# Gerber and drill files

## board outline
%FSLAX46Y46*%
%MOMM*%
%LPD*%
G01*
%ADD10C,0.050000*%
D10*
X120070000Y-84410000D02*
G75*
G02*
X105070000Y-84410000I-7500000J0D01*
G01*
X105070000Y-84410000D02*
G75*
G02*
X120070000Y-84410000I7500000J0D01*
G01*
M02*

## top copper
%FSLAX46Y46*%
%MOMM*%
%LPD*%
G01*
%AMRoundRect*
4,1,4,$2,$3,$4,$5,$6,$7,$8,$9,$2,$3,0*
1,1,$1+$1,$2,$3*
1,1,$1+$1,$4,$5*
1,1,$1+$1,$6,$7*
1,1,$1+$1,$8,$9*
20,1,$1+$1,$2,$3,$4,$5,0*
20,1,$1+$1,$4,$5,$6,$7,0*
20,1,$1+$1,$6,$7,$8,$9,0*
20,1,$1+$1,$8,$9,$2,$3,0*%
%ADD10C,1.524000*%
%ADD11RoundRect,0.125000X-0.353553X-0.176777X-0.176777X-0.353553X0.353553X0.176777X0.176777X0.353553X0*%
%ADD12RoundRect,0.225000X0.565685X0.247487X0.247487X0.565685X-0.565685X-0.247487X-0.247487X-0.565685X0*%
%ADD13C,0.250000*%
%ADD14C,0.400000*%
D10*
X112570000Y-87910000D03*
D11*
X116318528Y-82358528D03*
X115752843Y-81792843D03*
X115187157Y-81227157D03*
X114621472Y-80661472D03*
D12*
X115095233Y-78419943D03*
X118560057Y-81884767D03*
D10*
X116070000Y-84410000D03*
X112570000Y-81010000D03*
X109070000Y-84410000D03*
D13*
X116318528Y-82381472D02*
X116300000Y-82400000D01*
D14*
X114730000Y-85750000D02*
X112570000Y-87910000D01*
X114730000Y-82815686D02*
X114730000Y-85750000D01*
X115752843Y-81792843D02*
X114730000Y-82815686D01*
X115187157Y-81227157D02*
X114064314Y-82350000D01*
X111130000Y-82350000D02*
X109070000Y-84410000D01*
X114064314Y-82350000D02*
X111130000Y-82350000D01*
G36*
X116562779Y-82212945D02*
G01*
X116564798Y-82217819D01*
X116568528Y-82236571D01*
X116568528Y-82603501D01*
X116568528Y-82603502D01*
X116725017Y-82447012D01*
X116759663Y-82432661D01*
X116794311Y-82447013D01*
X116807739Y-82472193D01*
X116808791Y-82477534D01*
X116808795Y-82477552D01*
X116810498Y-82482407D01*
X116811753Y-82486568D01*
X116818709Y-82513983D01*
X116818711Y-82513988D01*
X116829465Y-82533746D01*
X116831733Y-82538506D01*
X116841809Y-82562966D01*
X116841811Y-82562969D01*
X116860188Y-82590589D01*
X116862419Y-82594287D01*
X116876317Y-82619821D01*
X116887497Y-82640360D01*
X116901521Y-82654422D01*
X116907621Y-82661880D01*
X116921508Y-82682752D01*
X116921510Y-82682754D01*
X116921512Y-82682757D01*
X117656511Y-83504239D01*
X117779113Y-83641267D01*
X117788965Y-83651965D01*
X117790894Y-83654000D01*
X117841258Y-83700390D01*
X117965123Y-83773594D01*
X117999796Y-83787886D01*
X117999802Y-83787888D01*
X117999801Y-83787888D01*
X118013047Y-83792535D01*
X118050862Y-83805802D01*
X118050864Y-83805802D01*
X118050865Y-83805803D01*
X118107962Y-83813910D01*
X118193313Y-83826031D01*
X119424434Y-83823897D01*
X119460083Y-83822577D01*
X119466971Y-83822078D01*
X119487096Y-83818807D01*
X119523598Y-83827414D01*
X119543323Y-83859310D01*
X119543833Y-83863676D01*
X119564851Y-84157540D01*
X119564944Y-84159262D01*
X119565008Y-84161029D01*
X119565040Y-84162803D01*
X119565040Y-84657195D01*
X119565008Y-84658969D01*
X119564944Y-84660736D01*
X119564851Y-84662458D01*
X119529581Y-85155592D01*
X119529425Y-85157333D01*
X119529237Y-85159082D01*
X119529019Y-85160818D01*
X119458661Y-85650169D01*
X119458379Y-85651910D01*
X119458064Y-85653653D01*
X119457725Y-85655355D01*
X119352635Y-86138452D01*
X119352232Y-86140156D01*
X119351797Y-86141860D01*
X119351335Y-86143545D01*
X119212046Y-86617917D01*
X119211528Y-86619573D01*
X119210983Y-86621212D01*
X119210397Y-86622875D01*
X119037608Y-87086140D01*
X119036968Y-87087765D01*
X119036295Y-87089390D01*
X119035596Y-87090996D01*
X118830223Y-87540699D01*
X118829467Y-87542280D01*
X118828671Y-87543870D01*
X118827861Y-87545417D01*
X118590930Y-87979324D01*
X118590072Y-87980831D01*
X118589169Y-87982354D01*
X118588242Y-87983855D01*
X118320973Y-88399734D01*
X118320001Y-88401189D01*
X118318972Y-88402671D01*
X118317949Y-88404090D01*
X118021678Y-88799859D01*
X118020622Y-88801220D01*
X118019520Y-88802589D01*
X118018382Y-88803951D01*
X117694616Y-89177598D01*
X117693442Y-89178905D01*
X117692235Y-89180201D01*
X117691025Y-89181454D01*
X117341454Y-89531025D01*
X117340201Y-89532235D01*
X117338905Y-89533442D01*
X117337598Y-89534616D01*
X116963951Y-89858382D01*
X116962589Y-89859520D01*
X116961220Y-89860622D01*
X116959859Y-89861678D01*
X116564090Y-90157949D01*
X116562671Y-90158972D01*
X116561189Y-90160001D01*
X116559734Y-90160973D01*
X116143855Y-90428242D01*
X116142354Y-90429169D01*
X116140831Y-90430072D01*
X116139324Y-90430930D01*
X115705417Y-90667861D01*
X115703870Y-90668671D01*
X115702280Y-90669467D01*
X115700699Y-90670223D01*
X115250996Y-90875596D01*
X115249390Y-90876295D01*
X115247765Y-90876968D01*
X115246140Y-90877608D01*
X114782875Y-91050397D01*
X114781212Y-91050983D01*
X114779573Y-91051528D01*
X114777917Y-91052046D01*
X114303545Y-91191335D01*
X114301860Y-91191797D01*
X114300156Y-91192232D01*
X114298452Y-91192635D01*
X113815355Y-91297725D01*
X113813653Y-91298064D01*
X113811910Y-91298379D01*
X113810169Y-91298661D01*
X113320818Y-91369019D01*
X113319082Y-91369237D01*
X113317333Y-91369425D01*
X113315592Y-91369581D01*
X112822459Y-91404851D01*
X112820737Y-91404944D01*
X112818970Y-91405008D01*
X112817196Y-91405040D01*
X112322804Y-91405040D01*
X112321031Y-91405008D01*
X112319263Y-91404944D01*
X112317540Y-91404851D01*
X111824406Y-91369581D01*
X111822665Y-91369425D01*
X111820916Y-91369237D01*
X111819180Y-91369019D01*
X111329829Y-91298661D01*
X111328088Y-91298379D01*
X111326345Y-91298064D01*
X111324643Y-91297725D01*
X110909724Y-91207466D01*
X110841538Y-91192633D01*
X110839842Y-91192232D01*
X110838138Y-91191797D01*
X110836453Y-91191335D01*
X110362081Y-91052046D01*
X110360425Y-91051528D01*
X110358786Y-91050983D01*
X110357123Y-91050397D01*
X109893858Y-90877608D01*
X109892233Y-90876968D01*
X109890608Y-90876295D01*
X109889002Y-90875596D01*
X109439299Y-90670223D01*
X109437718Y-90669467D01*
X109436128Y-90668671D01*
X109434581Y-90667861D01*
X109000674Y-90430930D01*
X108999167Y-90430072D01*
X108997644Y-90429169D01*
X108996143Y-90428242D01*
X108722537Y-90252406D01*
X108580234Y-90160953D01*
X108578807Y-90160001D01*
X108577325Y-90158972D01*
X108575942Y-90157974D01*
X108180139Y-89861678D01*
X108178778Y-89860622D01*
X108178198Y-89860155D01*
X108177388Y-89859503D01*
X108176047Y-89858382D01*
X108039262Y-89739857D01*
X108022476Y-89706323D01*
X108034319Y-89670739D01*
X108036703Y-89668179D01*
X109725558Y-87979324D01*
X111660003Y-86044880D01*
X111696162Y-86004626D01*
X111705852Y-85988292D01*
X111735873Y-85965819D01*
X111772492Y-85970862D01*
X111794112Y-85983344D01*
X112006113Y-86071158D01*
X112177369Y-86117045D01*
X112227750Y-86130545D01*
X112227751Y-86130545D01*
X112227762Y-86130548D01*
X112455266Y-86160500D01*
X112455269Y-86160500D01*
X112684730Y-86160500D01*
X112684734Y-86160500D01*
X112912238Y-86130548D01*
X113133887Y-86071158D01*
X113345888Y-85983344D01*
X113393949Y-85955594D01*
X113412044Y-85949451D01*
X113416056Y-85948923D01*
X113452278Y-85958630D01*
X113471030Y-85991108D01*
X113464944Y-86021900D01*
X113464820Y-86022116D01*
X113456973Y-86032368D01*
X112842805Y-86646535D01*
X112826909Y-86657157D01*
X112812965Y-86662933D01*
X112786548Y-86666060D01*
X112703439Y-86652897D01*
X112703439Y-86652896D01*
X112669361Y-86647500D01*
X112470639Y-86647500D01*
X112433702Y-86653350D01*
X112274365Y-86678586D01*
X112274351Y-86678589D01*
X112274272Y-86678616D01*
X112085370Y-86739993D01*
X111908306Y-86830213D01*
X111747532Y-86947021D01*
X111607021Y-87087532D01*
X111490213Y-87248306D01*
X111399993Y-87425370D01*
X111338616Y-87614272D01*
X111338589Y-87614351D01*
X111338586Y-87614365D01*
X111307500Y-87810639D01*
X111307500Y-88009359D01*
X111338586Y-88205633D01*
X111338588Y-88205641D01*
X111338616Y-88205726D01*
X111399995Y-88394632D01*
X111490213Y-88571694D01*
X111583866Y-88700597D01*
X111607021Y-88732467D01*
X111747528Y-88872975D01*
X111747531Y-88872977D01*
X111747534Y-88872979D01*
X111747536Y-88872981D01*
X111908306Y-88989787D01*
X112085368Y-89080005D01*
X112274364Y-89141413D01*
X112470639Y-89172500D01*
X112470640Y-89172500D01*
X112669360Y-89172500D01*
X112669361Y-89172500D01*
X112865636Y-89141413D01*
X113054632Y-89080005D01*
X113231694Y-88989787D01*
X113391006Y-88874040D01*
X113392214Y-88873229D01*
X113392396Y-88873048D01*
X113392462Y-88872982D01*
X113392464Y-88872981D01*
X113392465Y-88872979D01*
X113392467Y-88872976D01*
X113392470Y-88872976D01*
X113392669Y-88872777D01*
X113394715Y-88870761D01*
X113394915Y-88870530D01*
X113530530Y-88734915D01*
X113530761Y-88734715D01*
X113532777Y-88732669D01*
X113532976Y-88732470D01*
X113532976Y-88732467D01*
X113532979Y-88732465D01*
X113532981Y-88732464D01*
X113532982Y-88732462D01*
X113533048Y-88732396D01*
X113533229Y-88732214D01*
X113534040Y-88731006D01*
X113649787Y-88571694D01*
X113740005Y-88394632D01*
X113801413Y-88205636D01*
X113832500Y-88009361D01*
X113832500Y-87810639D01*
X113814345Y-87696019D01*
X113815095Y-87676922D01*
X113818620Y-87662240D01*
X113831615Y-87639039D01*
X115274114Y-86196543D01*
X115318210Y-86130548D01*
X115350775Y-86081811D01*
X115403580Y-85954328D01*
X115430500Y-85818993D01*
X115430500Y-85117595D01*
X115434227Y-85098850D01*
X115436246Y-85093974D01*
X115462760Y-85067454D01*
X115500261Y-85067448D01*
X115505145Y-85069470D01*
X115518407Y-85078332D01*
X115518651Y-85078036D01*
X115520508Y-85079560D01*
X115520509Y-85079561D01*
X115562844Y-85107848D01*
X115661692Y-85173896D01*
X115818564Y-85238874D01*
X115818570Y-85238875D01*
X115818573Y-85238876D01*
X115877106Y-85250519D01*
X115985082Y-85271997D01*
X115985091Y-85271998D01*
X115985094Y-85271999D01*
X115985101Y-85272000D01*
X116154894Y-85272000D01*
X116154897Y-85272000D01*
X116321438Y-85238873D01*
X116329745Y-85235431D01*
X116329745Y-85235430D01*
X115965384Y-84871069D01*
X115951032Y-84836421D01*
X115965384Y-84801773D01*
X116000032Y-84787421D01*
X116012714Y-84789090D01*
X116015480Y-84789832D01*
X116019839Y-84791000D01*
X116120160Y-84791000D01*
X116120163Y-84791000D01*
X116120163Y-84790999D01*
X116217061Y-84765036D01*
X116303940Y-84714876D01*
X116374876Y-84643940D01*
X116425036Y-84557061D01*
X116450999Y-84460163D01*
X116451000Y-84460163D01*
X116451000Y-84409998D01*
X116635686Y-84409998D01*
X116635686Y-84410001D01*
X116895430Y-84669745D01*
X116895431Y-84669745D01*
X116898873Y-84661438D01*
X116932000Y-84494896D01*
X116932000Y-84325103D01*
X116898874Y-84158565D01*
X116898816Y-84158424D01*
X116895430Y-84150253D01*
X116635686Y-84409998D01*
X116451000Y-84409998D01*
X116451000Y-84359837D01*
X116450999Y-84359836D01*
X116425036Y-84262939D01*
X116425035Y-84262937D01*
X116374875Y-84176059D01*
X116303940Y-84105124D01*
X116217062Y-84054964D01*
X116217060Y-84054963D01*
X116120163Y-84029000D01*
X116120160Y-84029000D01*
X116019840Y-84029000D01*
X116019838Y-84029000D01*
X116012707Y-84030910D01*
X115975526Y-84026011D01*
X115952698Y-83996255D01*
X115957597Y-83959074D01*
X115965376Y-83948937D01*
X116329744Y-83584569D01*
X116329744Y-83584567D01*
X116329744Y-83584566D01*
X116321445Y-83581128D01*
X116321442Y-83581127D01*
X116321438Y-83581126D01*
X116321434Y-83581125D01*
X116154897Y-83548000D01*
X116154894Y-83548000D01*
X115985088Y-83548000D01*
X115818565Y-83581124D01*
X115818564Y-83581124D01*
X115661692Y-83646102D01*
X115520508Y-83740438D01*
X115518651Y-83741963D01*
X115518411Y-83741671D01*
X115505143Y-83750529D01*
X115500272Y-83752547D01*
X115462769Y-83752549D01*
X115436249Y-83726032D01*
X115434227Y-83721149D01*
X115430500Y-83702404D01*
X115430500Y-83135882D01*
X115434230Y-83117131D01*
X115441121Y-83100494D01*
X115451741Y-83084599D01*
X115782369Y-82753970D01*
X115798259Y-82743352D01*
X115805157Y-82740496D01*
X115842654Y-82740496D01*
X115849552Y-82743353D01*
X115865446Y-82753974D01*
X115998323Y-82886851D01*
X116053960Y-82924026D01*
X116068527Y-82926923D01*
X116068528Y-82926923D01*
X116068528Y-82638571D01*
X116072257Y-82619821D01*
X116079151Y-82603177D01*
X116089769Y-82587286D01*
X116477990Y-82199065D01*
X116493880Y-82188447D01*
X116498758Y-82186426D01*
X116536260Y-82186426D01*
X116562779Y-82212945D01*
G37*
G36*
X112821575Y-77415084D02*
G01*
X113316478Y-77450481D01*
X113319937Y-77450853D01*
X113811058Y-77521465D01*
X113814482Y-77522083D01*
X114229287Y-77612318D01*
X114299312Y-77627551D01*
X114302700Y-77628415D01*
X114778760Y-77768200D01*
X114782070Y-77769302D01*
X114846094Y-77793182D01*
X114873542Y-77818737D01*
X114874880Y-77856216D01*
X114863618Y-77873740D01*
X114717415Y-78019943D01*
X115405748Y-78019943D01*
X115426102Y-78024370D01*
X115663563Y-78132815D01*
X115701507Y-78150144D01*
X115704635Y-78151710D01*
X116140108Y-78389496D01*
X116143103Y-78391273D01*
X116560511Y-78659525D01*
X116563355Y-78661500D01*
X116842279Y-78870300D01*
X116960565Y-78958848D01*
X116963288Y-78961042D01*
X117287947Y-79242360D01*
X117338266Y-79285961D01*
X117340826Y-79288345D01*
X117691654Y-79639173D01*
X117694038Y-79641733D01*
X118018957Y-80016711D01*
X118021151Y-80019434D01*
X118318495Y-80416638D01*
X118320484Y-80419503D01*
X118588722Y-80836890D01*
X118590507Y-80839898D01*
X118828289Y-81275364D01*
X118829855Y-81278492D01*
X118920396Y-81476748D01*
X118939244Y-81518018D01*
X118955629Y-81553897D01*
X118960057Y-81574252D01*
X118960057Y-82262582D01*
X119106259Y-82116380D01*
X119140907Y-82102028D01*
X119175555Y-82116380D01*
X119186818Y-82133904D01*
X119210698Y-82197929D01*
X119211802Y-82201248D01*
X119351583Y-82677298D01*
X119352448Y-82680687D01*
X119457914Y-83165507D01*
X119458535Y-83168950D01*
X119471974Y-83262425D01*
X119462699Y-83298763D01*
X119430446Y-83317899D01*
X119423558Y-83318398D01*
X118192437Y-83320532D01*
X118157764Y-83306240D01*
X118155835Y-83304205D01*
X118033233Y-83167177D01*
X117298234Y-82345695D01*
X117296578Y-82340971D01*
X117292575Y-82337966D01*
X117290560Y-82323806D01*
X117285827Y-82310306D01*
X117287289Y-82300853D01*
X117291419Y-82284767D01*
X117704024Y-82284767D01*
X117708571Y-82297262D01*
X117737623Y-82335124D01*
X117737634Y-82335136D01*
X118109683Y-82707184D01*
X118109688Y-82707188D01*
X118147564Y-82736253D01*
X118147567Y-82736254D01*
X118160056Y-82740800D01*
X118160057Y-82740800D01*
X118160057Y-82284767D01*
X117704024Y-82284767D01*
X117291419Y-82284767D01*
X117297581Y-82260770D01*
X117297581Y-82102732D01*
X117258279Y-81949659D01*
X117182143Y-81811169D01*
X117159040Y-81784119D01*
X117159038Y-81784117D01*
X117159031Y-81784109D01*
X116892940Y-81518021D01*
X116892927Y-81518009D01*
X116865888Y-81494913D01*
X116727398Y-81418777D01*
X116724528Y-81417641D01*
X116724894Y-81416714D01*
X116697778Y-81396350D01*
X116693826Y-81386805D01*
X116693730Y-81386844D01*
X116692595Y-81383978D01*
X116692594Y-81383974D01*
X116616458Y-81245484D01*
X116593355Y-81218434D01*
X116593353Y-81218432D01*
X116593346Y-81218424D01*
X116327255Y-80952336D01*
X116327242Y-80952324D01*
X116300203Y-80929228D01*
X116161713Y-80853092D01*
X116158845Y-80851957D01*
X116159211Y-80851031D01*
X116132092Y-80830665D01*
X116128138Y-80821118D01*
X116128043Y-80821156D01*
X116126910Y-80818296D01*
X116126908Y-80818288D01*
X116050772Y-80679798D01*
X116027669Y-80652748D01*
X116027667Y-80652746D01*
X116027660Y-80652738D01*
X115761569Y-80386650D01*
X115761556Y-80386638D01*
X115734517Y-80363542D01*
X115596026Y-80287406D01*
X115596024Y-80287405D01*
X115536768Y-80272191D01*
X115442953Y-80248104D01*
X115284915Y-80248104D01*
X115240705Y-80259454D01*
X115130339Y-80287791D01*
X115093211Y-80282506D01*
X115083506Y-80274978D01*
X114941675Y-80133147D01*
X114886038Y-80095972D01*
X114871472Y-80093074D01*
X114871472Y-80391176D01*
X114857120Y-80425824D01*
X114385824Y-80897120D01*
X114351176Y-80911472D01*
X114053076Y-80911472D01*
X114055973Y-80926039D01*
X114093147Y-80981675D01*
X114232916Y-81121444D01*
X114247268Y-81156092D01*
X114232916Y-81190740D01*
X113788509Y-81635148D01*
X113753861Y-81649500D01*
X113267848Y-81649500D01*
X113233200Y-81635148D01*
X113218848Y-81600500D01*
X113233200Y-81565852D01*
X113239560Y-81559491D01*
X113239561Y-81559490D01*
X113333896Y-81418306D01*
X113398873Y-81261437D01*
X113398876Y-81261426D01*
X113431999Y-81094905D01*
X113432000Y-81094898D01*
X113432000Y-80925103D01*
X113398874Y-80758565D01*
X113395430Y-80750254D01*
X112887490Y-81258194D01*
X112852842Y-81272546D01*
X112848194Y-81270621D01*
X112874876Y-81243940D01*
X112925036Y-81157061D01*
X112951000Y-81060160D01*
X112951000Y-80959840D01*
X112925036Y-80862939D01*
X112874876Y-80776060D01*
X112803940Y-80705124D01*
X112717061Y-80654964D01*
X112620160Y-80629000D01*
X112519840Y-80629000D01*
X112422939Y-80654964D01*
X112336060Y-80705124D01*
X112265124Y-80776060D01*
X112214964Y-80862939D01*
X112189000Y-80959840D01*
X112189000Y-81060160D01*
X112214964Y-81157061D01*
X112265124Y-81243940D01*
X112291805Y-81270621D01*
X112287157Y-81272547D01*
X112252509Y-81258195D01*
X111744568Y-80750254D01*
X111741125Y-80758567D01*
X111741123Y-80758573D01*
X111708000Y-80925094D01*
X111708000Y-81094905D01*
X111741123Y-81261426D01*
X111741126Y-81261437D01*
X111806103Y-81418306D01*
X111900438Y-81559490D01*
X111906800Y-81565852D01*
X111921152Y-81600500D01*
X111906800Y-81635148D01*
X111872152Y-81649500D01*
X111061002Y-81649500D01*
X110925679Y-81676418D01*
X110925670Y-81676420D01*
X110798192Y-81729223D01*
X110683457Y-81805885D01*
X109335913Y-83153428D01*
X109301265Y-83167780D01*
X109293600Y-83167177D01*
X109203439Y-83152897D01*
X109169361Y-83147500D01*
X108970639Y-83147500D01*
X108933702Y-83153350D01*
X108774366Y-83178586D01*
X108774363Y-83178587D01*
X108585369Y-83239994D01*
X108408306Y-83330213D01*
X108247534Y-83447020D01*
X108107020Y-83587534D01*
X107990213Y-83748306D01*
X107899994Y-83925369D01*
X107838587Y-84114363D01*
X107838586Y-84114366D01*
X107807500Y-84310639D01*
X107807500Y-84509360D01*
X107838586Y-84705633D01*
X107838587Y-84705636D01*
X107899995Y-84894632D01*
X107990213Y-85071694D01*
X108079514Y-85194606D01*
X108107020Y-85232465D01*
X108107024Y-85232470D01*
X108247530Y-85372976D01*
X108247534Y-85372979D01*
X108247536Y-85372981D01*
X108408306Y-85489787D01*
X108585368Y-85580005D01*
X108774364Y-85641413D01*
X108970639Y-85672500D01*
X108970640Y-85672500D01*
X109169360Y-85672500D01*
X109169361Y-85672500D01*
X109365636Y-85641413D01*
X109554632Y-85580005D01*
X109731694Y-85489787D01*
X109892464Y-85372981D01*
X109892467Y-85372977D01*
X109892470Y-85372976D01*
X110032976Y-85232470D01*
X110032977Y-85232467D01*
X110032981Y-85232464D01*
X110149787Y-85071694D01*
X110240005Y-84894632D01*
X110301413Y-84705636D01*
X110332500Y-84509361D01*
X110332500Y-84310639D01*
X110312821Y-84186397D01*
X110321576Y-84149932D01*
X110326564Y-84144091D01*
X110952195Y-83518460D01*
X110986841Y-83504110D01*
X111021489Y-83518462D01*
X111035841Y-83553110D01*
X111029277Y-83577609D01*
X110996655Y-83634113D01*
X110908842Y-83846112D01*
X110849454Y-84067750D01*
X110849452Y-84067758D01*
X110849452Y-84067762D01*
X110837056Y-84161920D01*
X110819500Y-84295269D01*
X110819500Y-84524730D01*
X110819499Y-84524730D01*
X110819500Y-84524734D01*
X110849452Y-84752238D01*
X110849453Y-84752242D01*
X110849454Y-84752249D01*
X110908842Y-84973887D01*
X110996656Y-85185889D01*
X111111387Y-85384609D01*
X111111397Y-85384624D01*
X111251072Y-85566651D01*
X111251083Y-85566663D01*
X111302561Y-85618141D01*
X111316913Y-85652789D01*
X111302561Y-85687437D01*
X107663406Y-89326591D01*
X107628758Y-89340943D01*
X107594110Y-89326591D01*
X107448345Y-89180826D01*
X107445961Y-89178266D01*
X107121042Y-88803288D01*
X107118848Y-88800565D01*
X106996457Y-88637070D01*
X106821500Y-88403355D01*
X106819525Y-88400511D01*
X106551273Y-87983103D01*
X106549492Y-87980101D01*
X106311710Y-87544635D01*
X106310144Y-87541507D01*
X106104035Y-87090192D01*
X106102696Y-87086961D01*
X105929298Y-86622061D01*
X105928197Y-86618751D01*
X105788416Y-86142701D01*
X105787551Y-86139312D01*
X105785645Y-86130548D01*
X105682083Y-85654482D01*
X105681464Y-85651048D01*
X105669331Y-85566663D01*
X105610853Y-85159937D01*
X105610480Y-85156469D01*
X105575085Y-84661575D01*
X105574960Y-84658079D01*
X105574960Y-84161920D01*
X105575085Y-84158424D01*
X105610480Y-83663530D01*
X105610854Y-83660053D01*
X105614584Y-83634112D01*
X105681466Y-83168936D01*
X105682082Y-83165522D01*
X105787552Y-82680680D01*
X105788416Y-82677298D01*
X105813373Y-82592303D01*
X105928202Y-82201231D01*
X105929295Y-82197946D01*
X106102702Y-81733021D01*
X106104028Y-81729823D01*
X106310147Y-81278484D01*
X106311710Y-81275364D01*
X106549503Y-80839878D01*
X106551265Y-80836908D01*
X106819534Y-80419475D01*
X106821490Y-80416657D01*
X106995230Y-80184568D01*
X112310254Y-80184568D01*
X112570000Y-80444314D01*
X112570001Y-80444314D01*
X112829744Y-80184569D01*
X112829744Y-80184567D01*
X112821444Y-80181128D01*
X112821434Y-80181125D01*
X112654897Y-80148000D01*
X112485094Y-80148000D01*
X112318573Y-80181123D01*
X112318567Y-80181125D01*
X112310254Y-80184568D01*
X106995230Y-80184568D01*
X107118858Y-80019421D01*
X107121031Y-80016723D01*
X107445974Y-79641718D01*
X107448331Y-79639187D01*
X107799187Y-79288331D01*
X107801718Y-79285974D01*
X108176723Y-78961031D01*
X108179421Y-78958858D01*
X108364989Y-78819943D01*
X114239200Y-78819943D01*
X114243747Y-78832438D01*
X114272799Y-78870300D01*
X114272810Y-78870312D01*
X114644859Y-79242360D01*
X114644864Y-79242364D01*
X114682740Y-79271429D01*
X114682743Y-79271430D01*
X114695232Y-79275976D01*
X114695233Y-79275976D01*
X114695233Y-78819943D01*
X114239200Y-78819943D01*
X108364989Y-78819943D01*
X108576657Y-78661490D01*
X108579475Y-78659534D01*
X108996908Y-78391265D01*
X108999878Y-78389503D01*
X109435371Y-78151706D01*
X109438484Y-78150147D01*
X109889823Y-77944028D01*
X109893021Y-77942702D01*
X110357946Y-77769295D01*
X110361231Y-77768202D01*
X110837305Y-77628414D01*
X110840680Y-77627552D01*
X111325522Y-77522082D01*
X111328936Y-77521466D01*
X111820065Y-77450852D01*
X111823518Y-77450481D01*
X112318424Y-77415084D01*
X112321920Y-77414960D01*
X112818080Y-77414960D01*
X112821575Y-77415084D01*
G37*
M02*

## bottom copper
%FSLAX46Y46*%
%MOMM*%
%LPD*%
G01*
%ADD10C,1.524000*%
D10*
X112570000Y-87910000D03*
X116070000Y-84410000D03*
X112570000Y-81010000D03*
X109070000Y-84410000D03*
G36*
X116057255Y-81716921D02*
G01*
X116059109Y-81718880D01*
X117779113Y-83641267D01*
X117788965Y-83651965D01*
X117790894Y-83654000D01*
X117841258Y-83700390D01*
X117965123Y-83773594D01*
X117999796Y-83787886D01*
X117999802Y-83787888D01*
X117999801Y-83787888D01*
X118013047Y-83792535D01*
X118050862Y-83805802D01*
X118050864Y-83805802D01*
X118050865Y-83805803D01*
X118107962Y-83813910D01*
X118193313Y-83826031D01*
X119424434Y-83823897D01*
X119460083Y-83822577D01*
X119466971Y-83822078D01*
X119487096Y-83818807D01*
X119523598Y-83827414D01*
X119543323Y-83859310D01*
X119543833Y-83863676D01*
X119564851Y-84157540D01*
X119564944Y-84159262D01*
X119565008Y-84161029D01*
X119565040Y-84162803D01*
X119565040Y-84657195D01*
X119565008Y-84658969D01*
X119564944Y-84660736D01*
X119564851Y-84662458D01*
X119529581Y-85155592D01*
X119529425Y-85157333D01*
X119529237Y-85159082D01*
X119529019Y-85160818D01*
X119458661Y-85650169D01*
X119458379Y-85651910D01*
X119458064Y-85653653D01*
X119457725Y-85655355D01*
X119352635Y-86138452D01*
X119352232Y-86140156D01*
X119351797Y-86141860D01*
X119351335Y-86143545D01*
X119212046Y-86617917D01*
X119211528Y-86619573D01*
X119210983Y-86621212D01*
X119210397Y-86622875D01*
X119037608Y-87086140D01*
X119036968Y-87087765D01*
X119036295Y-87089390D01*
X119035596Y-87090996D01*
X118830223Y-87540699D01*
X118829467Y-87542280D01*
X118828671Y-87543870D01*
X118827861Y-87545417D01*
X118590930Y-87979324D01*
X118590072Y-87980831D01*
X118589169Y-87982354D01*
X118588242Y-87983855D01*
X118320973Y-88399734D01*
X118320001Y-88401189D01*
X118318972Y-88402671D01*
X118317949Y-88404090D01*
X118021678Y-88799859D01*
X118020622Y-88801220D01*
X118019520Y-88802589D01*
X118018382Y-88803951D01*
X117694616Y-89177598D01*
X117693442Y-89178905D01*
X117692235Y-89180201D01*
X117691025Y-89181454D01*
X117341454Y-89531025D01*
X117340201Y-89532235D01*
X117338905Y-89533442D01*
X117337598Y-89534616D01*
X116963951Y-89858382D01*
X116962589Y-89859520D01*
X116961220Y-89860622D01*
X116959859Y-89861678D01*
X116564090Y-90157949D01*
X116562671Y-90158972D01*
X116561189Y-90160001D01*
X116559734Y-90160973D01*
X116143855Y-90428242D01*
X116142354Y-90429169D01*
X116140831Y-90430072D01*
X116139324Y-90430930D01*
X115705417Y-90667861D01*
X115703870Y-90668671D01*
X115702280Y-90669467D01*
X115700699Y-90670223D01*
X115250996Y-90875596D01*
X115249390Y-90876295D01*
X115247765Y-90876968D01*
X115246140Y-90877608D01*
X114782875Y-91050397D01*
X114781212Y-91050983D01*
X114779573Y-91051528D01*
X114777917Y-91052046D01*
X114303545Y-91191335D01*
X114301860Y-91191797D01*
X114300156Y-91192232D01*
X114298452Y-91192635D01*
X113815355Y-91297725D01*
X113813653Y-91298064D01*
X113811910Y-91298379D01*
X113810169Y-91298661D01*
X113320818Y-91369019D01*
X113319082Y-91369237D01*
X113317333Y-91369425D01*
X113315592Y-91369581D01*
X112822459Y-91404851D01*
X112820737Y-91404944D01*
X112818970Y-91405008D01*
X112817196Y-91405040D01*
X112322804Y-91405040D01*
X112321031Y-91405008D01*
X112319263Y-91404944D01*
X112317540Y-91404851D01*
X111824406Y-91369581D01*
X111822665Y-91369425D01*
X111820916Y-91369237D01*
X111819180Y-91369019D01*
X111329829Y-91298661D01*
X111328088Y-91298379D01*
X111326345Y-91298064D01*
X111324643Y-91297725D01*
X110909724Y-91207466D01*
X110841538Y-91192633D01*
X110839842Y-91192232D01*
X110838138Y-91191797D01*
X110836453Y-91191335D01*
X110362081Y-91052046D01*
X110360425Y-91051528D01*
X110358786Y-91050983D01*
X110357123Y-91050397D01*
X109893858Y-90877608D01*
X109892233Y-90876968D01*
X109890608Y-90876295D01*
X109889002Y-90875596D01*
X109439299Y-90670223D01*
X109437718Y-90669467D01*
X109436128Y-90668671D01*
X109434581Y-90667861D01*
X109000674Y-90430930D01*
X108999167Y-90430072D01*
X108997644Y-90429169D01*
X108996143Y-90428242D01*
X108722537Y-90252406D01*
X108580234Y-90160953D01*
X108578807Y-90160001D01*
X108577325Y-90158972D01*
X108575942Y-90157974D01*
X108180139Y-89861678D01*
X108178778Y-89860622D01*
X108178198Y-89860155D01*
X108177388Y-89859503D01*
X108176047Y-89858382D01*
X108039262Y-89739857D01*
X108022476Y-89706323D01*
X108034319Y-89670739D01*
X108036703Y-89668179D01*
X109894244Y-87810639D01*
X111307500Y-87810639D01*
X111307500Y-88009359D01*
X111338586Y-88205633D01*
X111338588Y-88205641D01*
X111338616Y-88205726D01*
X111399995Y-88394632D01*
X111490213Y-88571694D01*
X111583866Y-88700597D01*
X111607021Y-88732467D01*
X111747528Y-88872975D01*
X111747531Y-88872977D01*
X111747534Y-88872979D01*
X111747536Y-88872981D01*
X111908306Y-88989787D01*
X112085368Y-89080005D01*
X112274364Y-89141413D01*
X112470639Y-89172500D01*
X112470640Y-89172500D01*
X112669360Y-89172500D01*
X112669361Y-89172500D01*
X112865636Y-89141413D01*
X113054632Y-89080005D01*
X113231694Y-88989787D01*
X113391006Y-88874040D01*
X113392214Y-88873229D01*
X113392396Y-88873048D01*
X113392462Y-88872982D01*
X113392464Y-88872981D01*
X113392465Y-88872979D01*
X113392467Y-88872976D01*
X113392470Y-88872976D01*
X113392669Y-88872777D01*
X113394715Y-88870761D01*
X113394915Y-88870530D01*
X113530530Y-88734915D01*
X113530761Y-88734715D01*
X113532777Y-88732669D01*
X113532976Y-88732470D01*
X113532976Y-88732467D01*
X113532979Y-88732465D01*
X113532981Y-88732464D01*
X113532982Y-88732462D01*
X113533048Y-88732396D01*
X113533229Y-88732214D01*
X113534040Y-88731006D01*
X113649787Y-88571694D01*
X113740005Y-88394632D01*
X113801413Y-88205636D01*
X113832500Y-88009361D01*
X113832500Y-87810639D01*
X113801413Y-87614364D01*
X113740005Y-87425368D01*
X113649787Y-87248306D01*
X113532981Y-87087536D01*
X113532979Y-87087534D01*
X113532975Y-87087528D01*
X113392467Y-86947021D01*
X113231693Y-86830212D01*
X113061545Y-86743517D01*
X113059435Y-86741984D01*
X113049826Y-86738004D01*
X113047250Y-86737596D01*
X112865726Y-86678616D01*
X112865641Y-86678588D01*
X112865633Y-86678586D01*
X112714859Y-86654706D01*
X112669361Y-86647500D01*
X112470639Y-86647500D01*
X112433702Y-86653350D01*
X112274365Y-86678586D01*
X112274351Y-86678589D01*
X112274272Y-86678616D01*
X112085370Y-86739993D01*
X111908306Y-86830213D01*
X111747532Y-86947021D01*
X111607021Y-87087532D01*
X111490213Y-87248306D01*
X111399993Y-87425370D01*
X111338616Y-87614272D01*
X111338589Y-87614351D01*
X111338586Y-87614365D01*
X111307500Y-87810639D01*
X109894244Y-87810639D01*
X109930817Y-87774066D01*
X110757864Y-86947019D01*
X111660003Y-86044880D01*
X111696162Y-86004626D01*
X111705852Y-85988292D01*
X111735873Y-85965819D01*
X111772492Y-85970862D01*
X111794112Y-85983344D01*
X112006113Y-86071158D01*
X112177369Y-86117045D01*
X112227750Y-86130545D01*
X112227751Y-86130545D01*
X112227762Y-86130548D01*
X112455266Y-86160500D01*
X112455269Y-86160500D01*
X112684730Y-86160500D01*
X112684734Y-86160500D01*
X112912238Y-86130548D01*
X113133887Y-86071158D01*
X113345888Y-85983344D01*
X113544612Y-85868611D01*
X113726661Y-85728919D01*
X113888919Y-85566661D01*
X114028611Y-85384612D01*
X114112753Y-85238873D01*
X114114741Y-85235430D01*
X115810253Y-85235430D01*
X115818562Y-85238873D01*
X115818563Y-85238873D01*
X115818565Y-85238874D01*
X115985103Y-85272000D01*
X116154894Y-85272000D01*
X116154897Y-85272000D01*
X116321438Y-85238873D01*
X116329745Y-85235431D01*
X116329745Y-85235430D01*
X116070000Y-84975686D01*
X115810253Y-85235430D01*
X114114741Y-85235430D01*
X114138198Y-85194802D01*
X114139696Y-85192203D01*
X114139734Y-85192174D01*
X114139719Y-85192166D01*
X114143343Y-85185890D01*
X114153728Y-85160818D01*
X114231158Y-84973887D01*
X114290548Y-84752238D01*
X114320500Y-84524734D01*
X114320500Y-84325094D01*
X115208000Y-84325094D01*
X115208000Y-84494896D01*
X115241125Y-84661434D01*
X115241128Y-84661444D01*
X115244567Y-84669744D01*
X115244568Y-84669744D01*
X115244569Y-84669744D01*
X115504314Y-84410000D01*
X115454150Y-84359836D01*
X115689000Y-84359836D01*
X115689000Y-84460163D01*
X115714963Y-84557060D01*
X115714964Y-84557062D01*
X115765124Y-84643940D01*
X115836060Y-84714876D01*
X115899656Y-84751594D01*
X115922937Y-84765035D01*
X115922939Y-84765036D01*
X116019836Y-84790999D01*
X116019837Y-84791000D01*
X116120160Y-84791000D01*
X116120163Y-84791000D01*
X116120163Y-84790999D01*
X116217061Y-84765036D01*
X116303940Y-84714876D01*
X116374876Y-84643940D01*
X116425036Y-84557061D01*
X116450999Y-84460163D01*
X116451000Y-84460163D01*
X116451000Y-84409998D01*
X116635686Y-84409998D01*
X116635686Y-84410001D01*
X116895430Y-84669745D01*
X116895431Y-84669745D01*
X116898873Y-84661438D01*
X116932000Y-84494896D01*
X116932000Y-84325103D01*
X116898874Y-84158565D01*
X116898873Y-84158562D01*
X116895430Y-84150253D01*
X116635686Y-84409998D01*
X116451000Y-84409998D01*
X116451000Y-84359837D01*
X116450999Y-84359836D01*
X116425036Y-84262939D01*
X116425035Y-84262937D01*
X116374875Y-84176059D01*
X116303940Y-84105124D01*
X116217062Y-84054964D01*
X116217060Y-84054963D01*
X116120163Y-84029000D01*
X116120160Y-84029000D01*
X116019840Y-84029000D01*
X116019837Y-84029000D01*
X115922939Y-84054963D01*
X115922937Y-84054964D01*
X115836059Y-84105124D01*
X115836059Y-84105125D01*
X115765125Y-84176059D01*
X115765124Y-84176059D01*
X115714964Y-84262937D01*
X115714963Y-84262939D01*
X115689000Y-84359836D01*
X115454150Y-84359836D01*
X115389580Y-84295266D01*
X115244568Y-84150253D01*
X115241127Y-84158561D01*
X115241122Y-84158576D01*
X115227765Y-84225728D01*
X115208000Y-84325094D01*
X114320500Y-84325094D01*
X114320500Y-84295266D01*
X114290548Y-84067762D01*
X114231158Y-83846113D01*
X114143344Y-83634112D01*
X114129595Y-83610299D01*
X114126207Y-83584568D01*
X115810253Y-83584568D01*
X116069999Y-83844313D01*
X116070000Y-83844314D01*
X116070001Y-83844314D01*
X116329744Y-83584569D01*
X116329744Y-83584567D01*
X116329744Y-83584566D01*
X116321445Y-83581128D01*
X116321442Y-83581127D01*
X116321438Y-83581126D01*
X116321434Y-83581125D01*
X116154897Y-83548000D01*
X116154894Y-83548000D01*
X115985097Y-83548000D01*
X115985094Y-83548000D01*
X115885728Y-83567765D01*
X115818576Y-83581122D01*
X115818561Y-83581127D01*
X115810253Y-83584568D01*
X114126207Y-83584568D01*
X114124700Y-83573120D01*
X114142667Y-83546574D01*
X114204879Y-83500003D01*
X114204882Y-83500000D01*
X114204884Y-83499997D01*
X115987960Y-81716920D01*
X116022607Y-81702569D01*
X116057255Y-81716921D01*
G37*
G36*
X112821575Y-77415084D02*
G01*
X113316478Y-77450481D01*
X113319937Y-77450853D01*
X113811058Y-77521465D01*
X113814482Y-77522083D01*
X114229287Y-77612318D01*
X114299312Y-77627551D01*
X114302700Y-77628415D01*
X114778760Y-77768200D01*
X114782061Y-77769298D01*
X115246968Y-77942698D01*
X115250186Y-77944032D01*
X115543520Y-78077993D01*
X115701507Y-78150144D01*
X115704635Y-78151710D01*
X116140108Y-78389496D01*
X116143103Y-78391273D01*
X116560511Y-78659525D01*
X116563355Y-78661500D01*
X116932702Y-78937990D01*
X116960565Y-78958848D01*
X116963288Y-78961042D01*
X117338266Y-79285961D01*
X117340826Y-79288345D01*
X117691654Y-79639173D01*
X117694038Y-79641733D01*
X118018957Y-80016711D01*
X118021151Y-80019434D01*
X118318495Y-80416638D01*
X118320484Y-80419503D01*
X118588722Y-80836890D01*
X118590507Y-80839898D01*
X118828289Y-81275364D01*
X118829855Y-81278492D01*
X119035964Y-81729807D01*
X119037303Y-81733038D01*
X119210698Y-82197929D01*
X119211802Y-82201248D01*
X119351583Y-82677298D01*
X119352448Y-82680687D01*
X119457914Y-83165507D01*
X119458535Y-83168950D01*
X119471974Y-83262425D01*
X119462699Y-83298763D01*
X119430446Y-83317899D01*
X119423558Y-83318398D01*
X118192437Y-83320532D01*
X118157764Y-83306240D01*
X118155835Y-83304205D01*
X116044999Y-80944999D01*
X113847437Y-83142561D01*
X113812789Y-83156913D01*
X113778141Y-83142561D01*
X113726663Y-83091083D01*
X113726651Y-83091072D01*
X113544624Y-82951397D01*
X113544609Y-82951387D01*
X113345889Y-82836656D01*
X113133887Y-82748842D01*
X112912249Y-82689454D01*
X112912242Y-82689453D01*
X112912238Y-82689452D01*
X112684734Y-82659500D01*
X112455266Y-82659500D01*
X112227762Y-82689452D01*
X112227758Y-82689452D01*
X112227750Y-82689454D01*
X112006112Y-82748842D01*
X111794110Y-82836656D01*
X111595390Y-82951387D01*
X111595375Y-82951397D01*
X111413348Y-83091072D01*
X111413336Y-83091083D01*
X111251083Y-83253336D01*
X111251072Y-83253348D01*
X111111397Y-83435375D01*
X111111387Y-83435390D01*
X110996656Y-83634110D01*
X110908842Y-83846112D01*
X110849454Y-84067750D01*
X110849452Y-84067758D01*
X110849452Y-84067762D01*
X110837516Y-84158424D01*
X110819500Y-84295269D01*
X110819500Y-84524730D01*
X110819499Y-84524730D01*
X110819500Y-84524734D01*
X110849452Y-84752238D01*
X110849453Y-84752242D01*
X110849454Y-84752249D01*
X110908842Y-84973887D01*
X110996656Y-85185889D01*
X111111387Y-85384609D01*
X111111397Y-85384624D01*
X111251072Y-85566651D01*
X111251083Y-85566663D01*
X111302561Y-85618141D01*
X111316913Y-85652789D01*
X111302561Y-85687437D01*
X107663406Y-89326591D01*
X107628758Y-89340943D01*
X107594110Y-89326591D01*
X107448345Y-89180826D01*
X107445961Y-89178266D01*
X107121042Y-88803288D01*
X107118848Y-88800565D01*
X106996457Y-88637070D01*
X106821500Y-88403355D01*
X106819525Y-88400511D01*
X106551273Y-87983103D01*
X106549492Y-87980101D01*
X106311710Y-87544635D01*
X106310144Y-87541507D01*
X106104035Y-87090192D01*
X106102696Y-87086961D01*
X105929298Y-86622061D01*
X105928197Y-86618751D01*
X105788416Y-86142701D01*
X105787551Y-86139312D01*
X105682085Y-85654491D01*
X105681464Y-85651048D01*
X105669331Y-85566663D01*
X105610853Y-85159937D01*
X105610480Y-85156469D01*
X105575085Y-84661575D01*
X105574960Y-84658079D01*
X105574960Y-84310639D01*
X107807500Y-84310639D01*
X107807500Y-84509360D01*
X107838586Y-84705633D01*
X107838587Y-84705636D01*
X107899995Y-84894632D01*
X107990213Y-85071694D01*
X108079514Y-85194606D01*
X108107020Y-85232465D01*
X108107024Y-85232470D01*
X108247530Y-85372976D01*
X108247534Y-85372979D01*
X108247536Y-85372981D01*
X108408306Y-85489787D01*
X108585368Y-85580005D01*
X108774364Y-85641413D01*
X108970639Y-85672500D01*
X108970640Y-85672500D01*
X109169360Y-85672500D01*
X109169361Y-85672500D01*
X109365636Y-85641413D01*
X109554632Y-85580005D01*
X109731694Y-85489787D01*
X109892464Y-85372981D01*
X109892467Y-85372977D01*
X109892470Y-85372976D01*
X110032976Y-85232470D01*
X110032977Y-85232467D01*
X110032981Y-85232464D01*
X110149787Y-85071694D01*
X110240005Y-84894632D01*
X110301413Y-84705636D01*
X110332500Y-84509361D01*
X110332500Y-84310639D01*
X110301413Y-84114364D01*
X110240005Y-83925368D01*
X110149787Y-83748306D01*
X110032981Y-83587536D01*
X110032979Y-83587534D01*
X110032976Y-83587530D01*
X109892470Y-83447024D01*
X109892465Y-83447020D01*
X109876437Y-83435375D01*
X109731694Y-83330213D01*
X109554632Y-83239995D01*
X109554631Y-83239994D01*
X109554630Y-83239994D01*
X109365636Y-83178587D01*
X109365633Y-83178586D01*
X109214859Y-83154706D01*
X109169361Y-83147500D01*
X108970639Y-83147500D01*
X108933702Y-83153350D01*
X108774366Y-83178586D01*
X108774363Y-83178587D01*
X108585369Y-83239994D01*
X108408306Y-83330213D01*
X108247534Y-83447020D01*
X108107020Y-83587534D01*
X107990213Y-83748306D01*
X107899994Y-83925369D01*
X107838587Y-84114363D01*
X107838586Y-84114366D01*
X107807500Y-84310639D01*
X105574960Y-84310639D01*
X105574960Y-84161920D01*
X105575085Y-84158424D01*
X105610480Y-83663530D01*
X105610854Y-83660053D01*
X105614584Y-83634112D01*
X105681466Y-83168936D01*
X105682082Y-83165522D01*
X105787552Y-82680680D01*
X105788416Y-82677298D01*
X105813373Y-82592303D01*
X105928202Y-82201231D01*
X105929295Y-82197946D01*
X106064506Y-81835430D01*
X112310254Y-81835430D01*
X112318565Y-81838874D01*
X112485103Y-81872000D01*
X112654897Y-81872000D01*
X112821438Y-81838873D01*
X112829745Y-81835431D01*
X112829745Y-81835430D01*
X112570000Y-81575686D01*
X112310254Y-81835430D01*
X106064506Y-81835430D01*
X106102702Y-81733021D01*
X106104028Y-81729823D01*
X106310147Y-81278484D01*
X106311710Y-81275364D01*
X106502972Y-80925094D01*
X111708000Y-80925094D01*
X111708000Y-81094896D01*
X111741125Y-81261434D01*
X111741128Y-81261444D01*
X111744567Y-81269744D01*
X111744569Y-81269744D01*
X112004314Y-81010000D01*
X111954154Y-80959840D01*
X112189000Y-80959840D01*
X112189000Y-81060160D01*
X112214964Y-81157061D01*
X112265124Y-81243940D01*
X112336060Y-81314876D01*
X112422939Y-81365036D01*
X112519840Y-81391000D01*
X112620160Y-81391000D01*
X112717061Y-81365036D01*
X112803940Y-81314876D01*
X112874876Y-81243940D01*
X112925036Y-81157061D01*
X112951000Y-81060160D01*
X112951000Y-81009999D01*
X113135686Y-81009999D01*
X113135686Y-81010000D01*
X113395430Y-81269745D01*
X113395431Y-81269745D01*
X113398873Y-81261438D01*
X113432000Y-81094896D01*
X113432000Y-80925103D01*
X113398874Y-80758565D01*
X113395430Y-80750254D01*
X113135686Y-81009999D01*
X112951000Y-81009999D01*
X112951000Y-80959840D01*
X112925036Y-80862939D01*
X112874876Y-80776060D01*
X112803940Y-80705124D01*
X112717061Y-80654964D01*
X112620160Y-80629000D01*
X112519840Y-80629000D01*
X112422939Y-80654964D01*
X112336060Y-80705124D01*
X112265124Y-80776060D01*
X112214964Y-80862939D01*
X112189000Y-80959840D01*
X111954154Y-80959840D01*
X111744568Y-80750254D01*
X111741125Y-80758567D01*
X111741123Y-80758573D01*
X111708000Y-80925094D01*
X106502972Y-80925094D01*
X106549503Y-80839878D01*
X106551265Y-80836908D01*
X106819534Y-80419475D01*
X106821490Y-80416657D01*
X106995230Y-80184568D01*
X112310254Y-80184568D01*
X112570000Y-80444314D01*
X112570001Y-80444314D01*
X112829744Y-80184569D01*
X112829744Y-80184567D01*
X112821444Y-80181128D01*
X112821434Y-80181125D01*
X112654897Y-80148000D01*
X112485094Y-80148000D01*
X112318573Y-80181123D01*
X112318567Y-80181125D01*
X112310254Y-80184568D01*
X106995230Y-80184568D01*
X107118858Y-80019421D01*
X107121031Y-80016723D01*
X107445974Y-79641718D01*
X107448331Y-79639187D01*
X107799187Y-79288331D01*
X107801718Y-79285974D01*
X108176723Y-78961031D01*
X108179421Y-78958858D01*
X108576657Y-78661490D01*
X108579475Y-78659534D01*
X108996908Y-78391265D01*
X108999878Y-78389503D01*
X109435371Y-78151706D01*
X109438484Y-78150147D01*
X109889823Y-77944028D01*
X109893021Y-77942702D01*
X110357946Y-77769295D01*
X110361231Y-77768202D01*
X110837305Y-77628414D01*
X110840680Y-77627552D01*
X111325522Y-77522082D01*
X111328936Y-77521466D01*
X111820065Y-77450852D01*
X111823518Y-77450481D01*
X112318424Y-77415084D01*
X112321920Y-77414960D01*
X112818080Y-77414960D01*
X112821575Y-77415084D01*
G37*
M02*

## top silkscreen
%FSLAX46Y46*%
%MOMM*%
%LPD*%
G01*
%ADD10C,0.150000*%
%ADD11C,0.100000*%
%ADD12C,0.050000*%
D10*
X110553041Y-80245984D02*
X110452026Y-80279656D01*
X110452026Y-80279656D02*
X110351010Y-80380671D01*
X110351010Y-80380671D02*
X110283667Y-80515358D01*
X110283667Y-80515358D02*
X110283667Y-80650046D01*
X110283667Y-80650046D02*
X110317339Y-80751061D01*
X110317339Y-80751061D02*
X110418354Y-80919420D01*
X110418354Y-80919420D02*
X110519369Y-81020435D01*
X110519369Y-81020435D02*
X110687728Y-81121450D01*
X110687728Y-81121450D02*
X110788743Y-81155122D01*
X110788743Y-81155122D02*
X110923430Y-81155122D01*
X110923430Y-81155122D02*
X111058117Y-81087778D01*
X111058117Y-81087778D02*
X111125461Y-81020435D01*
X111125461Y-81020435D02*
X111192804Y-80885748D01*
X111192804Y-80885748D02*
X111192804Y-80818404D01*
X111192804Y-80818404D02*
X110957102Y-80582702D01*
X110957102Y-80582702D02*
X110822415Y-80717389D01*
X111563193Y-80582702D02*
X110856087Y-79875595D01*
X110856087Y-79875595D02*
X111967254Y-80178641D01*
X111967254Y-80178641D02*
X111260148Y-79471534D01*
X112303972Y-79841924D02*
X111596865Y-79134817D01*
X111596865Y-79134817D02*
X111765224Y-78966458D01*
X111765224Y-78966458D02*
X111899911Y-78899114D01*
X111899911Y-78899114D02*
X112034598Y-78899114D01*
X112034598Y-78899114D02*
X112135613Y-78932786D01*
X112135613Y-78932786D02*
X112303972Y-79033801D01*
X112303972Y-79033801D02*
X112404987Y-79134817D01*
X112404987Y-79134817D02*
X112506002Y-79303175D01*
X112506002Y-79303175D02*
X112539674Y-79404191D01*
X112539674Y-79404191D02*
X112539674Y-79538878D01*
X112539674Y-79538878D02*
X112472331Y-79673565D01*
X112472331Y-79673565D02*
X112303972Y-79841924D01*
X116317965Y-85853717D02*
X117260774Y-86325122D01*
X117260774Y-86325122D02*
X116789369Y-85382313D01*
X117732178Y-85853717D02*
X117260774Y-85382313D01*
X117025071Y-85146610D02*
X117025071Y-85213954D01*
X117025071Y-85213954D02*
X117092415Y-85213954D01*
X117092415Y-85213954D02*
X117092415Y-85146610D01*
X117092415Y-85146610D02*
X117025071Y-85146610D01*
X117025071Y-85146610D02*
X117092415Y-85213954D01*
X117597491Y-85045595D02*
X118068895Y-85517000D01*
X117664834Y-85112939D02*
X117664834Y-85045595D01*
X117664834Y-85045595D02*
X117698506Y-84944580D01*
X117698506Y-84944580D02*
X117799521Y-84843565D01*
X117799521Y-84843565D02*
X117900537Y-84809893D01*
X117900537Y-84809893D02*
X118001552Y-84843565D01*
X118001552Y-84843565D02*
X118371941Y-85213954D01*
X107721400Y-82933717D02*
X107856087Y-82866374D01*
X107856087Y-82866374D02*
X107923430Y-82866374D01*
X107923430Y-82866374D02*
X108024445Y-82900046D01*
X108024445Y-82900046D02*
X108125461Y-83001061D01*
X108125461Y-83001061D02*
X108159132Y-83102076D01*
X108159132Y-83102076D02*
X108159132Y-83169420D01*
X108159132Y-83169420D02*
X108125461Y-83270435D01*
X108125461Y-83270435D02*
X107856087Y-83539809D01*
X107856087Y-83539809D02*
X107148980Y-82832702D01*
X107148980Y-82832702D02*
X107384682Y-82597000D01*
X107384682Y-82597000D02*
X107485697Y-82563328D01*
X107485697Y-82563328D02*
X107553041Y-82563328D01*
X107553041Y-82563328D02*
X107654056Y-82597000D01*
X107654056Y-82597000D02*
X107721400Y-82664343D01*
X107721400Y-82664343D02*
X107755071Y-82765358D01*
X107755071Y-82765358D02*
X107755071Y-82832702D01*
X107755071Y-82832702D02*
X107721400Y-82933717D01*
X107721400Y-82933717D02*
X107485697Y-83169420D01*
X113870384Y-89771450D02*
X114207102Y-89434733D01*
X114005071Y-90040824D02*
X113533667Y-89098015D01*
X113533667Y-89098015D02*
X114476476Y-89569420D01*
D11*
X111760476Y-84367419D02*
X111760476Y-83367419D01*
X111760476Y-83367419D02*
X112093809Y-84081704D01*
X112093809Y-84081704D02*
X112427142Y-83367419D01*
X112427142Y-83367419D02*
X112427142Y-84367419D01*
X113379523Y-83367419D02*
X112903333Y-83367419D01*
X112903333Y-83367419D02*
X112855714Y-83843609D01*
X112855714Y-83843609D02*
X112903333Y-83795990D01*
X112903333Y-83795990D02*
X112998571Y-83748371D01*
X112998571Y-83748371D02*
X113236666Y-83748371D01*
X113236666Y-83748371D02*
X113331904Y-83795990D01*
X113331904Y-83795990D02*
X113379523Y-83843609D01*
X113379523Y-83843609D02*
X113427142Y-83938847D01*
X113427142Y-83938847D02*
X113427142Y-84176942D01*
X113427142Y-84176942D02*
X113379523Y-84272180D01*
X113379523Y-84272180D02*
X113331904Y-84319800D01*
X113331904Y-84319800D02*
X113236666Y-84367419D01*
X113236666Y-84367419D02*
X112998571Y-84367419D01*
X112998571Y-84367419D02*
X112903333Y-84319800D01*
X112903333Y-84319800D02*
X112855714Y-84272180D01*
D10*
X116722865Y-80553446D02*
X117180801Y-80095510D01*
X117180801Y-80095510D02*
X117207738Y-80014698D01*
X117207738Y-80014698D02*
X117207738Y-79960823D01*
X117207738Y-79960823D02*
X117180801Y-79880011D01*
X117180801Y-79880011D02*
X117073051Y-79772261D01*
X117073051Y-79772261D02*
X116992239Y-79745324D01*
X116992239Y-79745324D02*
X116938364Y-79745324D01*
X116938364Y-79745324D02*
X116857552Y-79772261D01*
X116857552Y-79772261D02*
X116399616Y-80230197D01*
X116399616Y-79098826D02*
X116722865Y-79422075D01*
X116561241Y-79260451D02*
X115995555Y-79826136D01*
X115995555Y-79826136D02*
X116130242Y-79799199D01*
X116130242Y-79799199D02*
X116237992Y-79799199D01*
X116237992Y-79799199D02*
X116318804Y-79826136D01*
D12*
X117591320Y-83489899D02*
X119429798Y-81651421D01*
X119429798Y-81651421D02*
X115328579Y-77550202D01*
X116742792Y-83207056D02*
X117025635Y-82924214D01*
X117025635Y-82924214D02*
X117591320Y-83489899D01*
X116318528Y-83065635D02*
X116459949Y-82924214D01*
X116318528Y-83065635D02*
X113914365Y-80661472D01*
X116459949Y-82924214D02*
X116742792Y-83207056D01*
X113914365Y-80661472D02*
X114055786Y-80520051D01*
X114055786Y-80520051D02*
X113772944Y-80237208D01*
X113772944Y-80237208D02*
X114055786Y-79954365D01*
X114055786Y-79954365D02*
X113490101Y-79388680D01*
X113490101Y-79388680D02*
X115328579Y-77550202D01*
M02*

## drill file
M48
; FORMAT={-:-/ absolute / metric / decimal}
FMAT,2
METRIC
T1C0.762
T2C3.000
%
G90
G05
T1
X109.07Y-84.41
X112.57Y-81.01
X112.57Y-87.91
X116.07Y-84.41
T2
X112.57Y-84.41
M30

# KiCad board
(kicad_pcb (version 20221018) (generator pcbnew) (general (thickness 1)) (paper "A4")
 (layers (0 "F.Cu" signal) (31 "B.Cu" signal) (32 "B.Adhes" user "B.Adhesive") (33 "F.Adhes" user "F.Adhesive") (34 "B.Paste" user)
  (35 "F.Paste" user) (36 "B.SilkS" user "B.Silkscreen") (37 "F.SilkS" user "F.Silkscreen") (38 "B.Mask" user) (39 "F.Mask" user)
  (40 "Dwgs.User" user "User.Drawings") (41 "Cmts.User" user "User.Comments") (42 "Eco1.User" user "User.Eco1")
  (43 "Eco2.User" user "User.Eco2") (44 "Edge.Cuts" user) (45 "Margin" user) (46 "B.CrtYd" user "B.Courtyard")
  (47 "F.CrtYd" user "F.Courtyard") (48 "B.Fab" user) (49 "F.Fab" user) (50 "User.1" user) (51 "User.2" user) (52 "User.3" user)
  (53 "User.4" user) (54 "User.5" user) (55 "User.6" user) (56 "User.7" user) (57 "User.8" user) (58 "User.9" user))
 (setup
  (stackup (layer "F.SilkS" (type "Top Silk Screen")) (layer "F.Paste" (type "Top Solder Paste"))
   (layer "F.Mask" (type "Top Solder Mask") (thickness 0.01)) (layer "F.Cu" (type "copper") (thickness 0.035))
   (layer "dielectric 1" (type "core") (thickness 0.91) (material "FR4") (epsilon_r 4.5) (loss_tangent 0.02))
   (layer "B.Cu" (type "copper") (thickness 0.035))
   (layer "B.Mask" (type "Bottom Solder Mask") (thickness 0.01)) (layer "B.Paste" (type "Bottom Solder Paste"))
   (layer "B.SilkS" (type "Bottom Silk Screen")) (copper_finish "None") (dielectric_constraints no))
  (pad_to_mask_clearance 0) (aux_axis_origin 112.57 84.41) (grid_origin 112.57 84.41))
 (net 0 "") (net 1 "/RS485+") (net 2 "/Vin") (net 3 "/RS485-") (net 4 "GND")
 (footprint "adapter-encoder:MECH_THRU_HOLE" (layer "F.Cu") (at 112.57 84.41)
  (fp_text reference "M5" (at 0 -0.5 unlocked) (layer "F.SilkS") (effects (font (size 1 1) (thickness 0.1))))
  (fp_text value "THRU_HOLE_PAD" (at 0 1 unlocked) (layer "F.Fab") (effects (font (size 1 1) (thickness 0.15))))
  (pad "" np_thru_hole circle (at 0 0) (size 3 3) (drill 3) (layers "F&B.Cu" "*.Mask")))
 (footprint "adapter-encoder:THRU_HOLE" (layer "F.Cu") (at 112.57 87.91 90)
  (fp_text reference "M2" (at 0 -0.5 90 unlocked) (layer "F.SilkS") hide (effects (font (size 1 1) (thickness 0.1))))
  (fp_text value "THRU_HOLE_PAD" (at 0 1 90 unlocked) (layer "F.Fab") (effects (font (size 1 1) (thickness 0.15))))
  (pad "1" thru_hole circle (at 0 0 90) (size 1.524 1.524) (drill 0.762) (layers "*.Cu" "*.Mask") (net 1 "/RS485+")))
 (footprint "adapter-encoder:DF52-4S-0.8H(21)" (layer "F.Cu") (at 115.47 81.51 135)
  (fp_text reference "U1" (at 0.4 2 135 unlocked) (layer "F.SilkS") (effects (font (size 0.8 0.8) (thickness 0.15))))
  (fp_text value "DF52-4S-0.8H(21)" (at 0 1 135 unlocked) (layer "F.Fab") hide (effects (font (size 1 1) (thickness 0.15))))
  (fp_line (start -2.9 0.1) (end -2.9 2.7) (stroke (width 0.05) (type default)) (layer "F.SilkS"))
  (fp_line (start -2.9 2.7) (end 2.9 2.7) (stroke (width 0.05) (type default)) (layer "F.SilkS"))
  (fp_line (start -2.1 -0.3) (end -2.1 0.1) (stroke (width 0.05) (type default)) (layer "F.SilkS"))
  (fp_line (start -2.1 0.1) (end -2.9 0.1) (stroke (width 0.05) (type default)) (layer "F.SilkS"))
  (fp_line (start -1.7 -0.5) (end -1.7 -0.3) (stroke (width 0.05) (type default)) (layer "F.SilkS"))
  (fp_line (start -1.7 -0.5) (end 1.7 -0.5) (stroke (width 0.05) (type default)) (layer "F.SilkS"))
  (fp_line (start -1.7 -0.3) (end -2.1 -0.3) (stroke (width 0.05) (type default)) (layer "F.SilkS"))
  (fp_line (start 1.7 -0.5) (end 1.7 -0.3) (stroke (width 0.05) (type default)) (layer "F.SilkS"))
  (fp_line (start 1.7 -0.3) (end 2.1 -0.3) (stroke (width 0.05) (type default)) (layer "F.SilkS"))
  (fp_line (start 2.1 -0.3) (end 2.1 0.1) (stroke (width 0.05) (type default)) (layer "F.SilkS"))
  (fp_line (start 2.1 0.1) (end 2.9 0.1) (stroke (width 0.05) (type default)) (layer "F.SilkS"))
  (fp_line (start 2.9 0.1) (end 2.9 2.7) (stroke (width 0.05) (type default)) (layer "F.SilkS"))
  (pad "1" smd roundrect (at -1.2 0 315) (size 0.5 1) (layers "F.Cu" "F.Paste" "F.Mask") (roundrect_rratio 0.25) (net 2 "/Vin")
   (thermal_bridge_angle 45))
  (pad "2" smd roundrect (at -0.4 0 315) (size 0.5 1) (layers "F.Cu" "F.Paste" "F.Mask") (roundrect_rratio 0.25) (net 1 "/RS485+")
   (thermal_bridge_angle 45))
  (pad "3" smd roundrect (at 0.4 0 315) (size 0.5 1) (layers "F.Cu" "F.Paste" "F.Mask") (roundrect_rratio 0.25) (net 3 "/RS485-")
   (thermal_bridge_angle 45))
  (pad "4" smd roundrect (at 1.2 0 315) (size 0.5 1) (layers "F.Cu" "F.Paste" "F.Mask") (roundrect_rratio 0.25) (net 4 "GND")
   (thermal_bridge_angle 45))
  (pad "5" smd roundrect (at 2.45 1.92 135) (size 0.9 1.6) (layers "F.Cu" "F.Paste" "F.Mask") (roundrect_rratio 0.25) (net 4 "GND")
   (solder_mask_margin 0.0508) (thermal_bridge_angle 45))
  (pad "6" smd roundrect (at -2.45 1.92 135) (size 0.9 1.6) (layers "F.Cu" "F.Paste" "F.Mask") (roundrect_rratio 0.25) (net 4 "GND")
   (solder_mask_margin 0.0508) (thermal_bridge_angle 45)))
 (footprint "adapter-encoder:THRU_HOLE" (layer "F.Cu") (at 116.07 84.41 180)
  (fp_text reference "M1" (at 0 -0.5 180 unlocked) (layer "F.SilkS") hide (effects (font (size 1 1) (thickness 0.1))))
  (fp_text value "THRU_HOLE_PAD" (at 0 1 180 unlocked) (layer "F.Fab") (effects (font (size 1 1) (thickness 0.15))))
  (pad "1" thru_hole circle (at 0 0 180) (size 1.524 1.524) (drill 0.762) (layers "*.Cu" "*.Mask") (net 2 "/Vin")))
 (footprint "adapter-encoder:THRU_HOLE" (layer "F.Cu") (at 112.57 81.01 -90)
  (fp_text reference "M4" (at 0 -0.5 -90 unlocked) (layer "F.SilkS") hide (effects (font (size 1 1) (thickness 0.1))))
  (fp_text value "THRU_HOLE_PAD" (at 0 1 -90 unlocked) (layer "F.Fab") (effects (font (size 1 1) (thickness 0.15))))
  (pad "1" thru_hole circle (at 0 0 270) (size 1.524 1.524) (drill 0.762) (layers "*.Cu" "*.Mask") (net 4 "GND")))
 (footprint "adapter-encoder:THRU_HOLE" (layer "F.Cu") (at 109.07 84.41)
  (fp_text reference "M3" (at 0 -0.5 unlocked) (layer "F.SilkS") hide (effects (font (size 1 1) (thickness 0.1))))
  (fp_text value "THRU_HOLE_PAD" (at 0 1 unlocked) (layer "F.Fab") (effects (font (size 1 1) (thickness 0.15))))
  (pad "1" thru_hole circle (at 0 0) (size 1.524 1.524) (drill 0.762) (layers "*.Cu" "*.Mask") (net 3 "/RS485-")))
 (gr_circle locked (center 112.57 84.41) (end 120.07 84.41) (stroke (width 0.05) (type default)) (fill none) (layer "Edge.Cuts"))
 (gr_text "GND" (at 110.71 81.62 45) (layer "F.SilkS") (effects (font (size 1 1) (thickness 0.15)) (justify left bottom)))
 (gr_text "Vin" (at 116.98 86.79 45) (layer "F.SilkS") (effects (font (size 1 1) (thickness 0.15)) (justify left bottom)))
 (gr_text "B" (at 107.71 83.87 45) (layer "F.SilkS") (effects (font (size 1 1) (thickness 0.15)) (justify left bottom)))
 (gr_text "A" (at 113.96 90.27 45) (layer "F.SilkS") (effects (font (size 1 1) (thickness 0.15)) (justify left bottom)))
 (segment (start 116.318528 82.381472) (end 116.3 82.4) (width 0.25) (layer "F.Cu") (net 2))
 (segment (start 114.73 85.75) (end 112.57 87.91) (width 0.4) (layer "F.Cu") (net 1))
 (segment (start 114.73 82.815686) (end 114.73 85.75) (width 0.4) (layer "F.Cu") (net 1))
 (segment (start 115.752843 81.792843) (end 114.73 82.815686) (width 0.4) (layer "F.Cu") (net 1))
 (segment (start 115.187157 81.227157) (end 114.064314 82.35) (width 0.4) (layer "F.Cu") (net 3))
 (segment (start 111.13 82.35) (end 109.07 84.41) (width 0.4) (layer "F.Cu") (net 3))
 (segment (start 114.064314 82.35) (end 111.13 82.35) (width 0.4) (layer "F.Cu") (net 3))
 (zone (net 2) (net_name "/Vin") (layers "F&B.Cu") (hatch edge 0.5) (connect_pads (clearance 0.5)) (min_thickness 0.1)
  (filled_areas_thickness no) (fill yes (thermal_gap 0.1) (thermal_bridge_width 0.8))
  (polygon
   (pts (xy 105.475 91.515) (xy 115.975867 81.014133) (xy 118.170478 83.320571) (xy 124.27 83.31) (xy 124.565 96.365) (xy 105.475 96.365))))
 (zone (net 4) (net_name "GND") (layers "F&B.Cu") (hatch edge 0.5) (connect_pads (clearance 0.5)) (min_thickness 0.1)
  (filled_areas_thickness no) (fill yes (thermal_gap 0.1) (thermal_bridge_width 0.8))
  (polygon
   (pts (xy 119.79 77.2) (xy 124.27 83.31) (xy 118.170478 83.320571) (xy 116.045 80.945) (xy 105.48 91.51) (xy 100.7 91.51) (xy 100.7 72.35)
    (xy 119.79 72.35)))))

